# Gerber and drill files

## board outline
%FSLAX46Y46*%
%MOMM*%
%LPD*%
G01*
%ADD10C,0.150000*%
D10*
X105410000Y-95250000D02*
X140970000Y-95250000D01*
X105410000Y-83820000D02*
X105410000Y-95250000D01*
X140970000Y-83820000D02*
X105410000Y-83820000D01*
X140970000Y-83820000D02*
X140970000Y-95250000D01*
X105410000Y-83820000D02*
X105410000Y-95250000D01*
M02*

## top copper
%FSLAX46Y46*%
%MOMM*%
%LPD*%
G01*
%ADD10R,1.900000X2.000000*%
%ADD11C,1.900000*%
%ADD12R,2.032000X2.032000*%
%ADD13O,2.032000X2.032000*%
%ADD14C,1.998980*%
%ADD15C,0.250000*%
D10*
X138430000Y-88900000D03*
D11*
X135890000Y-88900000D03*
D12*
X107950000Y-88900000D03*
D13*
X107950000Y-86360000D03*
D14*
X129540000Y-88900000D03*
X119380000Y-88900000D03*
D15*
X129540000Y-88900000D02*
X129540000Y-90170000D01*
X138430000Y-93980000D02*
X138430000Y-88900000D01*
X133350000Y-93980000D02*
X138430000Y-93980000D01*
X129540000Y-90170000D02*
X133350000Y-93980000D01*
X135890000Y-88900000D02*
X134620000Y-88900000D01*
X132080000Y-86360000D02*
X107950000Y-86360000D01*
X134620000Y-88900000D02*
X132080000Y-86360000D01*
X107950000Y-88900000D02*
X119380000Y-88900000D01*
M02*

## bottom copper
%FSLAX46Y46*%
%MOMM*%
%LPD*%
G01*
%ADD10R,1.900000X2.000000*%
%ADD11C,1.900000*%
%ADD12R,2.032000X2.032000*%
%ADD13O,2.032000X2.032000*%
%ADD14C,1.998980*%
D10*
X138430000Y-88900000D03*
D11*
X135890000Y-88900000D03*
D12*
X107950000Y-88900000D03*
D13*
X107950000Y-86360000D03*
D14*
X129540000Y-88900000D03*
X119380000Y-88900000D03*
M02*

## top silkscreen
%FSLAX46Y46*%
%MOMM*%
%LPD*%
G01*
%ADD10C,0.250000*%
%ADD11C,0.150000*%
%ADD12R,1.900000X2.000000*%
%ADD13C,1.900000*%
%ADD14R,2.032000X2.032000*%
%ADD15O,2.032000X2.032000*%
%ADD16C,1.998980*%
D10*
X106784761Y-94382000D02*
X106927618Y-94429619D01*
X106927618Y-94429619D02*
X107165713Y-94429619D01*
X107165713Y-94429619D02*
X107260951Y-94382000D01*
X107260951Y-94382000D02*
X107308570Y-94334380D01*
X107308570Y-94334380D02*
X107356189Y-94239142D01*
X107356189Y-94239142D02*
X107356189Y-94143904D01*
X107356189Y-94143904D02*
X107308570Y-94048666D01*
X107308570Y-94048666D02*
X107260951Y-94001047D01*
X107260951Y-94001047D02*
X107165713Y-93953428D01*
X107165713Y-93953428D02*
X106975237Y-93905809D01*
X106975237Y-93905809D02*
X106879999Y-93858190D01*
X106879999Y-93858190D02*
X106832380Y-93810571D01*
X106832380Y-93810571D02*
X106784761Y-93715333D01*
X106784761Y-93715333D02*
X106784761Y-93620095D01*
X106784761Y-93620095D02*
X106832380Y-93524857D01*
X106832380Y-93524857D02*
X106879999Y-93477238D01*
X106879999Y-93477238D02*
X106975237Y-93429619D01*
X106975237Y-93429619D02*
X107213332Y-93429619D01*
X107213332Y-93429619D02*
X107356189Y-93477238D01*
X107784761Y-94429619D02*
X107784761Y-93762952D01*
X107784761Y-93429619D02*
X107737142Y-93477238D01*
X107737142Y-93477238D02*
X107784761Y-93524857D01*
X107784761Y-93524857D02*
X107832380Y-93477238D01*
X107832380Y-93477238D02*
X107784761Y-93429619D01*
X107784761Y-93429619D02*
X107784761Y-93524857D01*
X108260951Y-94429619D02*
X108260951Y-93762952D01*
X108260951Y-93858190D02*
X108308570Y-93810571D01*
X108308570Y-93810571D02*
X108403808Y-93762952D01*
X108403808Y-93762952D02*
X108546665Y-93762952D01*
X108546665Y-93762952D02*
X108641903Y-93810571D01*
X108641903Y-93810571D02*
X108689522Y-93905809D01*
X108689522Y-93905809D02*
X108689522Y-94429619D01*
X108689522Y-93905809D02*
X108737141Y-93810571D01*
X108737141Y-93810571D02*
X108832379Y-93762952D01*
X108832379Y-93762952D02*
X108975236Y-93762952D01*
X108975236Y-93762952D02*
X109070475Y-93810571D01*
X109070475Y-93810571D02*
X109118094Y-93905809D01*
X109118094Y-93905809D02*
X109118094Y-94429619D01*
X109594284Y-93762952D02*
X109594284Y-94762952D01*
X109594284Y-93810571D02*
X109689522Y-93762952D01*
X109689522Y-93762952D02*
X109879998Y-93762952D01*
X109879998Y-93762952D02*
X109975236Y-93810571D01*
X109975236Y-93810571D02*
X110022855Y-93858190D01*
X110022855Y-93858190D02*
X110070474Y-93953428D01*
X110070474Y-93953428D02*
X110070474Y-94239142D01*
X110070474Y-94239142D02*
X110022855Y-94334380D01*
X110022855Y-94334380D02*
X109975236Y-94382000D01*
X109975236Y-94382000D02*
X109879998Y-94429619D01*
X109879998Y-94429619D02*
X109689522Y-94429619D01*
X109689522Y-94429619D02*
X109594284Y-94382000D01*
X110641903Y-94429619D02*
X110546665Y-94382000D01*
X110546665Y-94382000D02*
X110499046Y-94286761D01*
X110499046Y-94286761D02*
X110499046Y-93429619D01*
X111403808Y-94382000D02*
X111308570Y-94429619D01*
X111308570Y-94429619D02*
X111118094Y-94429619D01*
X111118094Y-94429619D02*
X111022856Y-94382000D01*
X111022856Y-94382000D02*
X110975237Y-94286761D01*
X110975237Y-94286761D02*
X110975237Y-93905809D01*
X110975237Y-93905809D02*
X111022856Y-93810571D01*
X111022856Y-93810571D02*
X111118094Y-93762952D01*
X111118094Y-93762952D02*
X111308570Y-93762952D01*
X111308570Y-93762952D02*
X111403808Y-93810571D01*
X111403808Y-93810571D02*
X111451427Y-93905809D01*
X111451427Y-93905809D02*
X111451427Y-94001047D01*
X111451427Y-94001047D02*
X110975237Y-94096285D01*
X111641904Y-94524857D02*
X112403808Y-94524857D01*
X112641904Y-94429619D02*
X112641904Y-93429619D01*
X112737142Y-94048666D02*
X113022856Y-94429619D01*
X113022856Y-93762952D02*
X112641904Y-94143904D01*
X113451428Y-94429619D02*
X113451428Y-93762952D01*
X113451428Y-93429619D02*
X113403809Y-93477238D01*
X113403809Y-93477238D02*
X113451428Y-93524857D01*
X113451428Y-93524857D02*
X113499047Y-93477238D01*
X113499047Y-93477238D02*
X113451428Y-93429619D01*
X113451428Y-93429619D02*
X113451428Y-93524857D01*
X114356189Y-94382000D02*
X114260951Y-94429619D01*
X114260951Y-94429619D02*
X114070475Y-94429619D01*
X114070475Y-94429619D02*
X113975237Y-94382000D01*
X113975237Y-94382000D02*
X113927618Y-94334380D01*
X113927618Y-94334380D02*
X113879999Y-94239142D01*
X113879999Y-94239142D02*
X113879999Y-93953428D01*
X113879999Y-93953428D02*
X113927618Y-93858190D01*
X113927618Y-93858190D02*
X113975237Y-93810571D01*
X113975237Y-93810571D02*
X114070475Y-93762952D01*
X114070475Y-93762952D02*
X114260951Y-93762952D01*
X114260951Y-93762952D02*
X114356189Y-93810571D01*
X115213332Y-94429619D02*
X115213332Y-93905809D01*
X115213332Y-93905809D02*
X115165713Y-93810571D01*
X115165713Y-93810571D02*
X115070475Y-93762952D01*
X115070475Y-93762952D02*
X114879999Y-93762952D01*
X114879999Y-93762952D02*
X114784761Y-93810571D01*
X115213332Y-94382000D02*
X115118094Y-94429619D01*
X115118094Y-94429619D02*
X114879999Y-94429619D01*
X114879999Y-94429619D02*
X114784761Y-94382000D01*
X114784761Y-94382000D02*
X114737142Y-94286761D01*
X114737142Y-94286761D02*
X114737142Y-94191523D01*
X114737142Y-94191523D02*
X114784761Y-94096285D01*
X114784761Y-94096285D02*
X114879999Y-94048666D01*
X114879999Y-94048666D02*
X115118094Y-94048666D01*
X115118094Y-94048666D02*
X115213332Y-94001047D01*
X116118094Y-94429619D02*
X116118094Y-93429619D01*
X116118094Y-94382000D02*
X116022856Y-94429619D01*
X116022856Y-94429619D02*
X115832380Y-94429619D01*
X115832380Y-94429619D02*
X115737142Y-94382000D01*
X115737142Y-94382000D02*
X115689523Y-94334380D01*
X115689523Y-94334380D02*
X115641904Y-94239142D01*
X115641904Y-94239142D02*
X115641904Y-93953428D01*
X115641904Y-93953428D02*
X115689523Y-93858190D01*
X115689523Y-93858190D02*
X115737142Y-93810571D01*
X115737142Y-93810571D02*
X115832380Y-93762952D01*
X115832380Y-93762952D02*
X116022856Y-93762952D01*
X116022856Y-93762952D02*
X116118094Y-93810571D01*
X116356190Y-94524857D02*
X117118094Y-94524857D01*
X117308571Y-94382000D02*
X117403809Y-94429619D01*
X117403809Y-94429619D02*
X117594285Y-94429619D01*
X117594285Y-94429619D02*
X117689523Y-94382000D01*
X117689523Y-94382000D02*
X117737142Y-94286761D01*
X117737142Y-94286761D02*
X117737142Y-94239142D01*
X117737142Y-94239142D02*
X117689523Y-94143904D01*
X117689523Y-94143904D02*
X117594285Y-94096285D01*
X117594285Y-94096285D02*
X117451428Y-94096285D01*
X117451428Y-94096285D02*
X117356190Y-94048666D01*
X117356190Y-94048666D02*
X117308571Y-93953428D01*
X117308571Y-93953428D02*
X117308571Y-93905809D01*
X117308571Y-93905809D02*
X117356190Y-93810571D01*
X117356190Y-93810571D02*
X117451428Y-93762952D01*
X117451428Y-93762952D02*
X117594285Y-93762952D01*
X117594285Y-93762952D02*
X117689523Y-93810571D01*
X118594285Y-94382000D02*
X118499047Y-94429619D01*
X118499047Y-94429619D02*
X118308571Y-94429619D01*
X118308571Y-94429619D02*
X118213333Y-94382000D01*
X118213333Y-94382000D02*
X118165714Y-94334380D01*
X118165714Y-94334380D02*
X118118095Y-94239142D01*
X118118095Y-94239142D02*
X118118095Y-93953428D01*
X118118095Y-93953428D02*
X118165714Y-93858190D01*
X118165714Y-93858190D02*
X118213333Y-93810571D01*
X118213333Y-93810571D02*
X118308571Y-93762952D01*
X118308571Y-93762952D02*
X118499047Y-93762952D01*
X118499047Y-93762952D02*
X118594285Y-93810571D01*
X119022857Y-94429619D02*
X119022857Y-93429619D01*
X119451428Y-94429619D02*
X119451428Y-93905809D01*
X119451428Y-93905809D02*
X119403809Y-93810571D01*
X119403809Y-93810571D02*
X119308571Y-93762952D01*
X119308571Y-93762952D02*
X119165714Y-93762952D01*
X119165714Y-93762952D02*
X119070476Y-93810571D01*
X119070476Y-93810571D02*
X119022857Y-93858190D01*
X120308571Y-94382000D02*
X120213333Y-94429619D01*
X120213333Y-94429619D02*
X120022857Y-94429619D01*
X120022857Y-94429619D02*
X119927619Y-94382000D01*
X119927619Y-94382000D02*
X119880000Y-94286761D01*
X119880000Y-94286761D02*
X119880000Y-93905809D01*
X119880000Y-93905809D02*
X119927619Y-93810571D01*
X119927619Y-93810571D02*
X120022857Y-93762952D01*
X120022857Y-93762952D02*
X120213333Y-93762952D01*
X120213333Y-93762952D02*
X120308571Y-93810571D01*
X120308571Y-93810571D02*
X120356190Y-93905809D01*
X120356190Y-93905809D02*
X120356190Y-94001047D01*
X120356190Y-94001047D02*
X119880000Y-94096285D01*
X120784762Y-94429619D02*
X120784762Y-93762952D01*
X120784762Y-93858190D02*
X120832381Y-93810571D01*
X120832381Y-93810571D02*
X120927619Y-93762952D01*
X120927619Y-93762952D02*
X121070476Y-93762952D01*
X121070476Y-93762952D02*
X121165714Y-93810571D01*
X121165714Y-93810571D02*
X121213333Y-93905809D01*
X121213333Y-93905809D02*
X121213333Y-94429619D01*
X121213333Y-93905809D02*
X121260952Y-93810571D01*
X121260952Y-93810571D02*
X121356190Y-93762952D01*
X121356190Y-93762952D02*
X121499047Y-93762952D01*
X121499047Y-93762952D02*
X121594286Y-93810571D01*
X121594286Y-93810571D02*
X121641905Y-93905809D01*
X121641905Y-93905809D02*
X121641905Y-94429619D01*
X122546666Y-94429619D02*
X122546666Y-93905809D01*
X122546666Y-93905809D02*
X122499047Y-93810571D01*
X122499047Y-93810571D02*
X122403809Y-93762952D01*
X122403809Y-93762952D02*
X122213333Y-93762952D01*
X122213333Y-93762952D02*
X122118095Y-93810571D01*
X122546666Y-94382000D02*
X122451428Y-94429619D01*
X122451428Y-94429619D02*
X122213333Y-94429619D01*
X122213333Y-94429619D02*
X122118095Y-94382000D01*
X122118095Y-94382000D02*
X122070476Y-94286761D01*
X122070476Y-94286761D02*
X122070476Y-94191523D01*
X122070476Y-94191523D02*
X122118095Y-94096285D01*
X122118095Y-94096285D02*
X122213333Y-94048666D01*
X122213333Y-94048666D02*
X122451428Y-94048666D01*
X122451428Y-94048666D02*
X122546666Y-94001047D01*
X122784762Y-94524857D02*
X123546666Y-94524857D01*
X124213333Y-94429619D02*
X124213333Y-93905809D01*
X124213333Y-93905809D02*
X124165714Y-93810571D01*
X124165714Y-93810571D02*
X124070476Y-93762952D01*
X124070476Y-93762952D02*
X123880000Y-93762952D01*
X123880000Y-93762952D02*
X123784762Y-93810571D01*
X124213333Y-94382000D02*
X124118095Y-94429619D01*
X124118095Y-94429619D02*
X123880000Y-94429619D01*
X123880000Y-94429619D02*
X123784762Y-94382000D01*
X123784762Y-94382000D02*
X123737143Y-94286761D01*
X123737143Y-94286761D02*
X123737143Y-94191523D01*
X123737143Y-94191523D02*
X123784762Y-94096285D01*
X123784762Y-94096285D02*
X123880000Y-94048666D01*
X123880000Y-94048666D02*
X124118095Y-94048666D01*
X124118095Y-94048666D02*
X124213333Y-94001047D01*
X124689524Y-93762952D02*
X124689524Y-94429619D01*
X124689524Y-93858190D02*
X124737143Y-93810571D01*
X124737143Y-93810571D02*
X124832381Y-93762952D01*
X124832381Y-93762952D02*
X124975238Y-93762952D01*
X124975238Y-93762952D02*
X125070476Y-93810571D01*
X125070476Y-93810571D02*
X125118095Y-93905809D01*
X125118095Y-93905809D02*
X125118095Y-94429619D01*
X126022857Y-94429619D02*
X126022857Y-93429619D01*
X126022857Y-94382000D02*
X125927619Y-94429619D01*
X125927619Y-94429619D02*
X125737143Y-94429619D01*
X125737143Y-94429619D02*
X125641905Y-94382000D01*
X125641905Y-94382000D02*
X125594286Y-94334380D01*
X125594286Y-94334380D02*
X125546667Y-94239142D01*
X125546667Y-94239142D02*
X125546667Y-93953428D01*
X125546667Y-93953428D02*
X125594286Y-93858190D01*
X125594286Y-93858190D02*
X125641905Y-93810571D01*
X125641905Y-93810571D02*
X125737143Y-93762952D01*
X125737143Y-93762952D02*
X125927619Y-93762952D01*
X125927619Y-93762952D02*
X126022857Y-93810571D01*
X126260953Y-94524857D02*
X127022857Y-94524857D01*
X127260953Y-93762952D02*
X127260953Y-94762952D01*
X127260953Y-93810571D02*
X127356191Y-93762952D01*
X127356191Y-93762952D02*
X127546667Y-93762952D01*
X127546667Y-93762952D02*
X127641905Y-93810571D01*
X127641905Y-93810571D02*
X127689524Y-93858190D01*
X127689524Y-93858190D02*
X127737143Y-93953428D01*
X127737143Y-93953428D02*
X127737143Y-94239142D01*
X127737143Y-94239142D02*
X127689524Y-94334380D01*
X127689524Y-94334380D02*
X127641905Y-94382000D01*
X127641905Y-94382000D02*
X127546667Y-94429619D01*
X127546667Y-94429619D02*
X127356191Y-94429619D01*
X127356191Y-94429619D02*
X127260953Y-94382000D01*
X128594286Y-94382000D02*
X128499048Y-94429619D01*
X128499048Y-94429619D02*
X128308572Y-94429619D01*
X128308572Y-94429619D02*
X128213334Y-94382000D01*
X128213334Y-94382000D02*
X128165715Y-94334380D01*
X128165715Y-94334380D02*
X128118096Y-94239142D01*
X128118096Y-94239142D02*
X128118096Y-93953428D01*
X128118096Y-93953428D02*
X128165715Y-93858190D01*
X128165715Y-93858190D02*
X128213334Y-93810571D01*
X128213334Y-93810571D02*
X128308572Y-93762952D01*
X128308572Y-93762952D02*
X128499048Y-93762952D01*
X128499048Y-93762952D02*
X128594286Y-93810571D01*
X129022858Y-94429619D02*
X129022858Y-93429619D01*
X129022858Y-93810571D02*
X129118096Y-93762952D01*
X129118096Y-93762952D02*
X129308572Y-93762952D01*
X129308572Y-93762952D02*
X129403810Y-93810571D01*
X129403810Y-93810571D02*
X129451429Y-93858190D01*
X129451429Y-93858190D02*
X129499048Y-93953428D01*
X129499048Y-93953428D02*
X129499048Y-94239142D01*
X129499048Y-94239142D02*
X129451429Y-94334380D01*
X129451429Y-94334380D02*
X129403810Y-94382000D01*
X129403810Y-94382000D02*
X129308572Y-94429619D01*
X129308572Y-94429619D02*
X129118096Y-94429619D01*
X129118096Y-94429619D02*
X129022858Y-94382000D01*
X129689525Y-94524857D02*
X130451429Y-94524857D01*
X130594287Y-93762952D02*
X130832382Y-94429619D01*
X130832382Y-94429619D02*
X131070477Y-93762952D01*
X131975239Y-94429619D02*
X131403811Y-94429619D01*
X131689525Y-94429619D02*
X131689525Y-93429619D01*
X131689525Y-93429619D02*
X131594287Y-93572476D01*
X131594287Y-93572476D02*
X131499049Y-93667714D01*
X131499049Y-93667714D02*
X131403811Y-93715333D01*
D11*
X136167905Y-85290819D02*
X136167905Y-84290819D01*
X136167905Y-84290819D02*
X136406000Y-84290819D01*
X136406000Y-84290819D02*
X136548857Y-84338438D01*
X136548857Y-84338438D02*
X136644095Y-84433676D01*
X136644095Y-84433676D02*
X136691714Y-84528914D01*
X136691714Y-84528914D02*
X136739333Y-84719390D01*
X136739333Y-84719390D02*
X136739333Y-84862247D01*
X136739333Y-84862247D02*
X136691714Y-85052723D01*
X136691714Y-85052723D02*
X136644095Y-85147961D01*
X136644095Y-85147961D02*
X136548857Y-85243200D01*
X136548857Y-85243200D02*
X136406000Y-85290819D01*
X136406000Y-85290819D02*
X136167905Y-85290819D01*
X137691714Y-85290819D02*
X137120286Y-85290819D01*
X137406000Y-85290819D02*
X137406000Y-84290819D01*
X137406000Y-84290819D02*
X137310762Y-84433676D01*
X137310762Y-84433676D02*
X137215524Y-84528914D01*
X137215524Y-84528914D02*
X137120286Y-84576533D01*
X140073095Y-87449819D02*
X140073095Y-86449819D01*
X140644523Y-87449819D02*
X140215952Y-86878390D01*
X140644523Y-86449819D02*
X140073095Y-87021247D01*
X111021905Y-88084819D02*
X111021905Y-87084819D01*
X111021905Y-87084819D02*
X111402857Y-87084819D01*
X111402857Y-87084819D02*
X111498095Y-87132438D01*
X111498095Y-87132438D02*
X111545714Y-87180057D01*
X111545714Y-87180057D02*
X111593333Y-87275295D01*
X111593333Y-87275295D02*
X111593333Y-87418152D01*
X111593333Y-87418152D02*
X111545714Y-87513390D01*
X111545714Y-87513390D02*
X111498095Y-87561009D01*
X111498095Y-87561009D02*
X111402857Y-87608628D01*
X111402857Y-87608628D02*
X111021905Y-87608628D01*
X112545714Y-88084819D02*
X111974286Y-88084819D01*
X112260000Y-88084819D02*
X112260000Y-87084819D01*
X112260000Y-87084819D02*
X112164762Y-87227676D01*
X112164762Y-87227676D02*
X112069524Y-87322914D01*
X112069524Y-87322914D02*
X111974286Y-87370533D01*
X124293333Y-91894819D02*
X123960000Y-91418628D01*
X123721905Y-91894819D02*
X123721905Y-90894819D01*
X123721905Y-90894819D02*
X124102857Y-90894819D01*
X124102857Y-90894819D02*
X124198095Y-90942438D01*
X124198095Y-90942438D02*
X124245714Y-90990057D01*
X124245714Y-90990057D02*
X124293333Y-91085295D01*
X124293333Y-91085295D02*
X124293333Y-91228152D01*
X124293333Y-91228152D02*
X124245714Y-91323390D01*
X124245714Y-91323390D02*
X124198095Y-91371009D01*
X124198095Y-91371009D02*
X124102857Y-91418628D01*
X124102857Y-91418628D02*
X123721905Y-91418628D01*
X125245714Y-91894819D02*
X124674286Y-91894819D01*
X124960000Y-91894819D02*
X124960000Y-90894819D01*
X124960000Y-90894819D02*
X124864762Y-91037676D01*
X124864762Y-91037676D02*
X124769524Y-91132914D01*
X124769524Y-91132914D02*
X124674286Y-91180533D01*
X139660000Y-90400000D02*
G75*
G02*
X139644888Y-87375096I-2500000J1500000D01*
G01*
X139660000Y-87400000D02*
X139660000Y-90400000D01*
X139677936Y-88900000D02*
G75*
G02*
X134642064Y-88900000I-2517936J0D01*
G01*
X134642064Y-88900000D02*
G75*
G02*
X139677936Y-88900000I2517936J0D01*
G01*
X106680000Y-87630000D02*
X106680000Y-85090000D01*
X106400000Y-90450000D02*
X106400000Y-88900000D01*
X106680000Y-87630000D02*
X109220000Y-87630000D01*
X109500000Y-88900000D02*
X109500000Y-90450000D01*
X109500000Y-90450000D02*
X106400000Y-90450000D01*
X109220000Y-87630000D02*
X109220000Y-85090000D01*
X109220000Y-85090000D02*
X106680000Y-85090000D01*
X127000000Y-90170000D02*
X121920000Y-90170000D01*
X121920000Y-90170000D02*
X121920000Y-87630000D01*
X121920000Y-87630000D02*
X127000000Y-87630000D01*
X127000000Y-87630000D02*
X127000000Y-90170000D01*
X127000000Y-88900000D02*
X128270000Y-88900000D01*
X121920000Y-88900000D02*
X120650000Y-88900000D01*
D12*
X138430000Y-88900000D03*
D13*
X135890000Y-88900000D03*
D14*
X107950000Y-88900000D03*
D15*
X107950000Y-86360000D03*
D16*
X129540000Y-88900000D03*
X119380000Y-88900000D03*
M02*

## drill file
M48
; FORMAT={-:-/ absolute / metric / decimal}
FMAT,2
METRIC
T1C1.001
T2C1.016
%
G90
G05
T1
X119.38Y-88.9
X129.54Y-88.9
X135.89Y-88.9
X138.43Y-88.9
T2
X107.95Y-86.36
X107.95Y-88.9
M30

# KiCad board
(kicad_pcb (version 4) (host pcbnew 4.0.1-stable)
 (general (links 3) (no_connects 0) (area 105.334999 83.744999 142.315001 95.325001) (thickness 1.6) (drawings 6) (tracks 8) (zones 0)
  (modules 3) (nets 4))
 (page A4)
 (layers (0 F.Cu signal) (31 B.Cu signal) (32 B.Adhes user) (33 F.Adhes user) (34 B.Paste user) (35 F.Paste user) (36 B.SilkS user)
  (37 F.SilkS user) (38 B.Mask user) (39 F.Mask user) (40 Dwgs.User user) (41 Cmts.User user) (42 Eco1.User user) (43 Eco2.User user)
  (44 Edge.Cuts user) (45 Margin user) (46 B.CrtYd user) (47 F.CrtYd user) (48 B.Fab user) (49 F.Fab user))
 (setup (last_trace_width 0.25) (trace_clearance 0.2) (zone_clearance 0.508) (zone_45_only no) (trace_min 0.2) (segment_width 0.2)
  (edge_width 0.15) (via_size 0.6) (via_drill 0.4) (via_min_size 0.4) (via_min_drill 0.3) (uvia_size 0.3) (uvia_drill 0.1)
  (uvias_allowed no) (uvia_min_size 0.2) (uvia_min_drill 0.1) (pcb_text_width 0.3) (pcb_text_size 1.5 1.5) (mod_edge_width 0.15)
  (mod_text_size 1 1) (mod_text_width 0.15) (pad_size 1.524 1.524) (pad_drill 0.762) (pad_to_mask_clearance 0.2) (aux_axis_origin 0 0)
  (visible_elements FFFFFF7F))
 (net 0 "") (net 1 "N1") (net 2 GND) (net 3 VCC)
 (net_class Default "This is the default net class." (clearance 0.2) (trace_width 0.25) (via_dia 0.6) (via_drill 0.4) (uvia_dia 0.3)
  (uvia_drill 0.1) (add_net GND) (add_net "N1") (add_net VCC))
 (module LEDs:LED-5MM (layer F.Cu) (at 138.43 88.9 180)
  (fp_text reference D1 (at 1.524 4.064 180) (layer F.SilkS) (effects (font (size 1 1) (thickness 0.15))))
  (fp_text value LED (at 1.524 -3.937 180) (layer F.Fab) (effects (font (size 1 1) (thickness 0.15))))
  (fp_arc (start 1.27 0) (end -1.23 -1.5) (angle 297.5) (layer F.SilkS) (width 0.15))
  (fp_line (start -1.23 1.5) (end -1.23 -1.5) (layer F.SilkS) (width 0.15))
  (fp_circle (center 1.27 0) (end 0.97 -2.5) (layer F.SilkS) (width 0.15))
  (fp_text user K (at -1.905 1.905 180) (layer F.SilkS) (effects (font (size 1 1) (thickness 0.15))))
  (pad 1 thru_hole rect (at 0 0 270) (size 2 1.9) (drill 1.00076) (layers *.Cu *.Mask F.SilkS) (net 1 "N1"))
  (pad 2 thru_hole circle (at 2.54 0 180) (size 1.9 1.9) (drill 1.00076) (layers *.Cu *.Mask F.SilkS) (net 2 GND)))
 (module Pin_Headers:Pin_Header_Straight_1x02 (layer F.Cu) (at 107.95 88.9 180)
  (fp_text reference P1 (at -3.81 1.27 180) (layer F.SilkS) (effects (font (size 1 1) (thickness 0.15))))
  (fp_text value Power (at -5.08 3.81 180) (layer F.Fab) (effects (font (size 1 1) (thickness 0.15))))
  (fp_line (start 1.27 1.27) (end 1.27 3.81) (layer F.SilkS) (width 0.15))
  (fp_line (start 1.55 -1.55) (end 1.55 0) (layer F.SilkS) (width 0.15))
  (fp_line (start 1.27 1.27) (end -1.27 1.27) (layer F.SilkS) (width 0.15))
  (fp_line (start -1.55 0) (end -1.55 -1.55) (layer F.SilkS) (width 0.15))
  (fp_line (start -1.55 -1.55) (end 1.55 -1.55) (layer F.SilkS) (width 0.15))
  (fp_line (start -1.27 1.27) (end -1.27 3.81) (layer F.SilkS) (width 0.15))
  (fp_line (start -1.27 3.81) (end 1.27 3.81) (layer F.SilkS) (width 0.15))
  (pad 1 thru_hole rect (at 0 0 180) (size 2.032 2.032) (drill 1.016) (layers *.Cu *.Mask F.SilkS) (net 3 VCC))
  (pad 2 thru_hole oval (at 0 2.54 180) (size 2.032 2.032) (drill 1.016) (layers *.Cu *.Mask F.SilkS) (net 2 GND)))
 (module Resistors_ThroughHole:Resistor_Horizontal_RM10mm (layer F.Cu) (at 124.46 88.9 180)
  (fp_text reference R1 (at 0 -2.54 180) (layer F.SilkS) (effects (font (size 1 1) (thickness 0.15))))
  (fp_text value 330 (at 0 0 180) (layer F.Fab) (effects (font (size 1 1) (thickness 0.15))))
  (fp_line (start -2.54 -1.27) (end 2.54 -1.27) (layer F.SilkS) (width 0.15))
  (fp_line (start 2.54 -1.27) (end 2.54 1.27) (layer F.SilkS) (width 0.15))
  (fp_line (start 2.54 1.27) (end -2.54 1.27) (layer F.SilkS) (width 0.15))
  (fp_line (start -2.54 1.27) (end -2.54 -1.27) (layer F.SilkS) (width 0.15))
  (fp_line (start -2.54 0) (end -3.81 0) (layer F.SilkS) (width 0.15))
  (fp_line (start 2.54 0) (end 3.81 0) (layer F.SilkS) (width 0.15))
  (pad 1 thru_hole circle (at -5.08 0 180) (size 1.99898 1.99898) (drill 1.00076) (layers *.Cu *.SilkS *.Mask) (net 1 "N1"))
  (pad 2 thru_hole circle (at 5.08 0 180) (size 1.99898 1.99898) (drill 1.00076) (layers *.Cu *.SilkS *.Mask) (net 3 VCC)))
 (gr_line (start 105.41 95.25) (end 140.97 95.25) (angle 90) (layer Edge.Cuts) (width 0.15))
 (gr_line (start 105.41 83.82) (end 105.41 95.25) (angle 90) (layer Edge.Cuts) (width 0.15))
 (gr_line (start 140.97 83.82) (end 105.41 83.82) (angle 90) (layer Edge.Cuts) (width 0.15))
 (gr_line (start 140.97 83.82) (end 140.97 95.25) (angle 90) (layer Edge.Cuts) (width 0.15))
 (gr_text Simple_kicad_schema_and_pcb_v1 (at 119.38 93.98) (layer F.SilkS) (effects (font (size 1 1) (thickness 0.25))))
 (gr_line (start 105.41 83.82) (end 105.41 95.25) (angle 90) (layer Edge.Cuts) (width 0.15))
 (segment (start 129.54 88.9) (end 129.54 90.17) (width 0.25) (layer F.Cu) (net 1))
 (segment (start 138.43 93.98) (end 138.43 88.9) (width 0.25) (layer F.Cu) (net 1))
 (segment (start 133.35 93.98) (end 138.43 93.98) (width 0.25) (layer F.Cu) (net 1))
 (segment (start 129.54 90.17) (end 133.35 93.98) (width 0.25) (layer F.Cu) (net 1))
 (segment (start 135.89 88.9) (end 134.62 88.9) (width 0.25) (layer F.Cu) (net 2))
 (segment (start 132.08 86.36) (end 107.95 86.36) (width 0.25) (layer F.Cu) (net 2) (status 20))
 (segment (start 134.62 88.9) (end 132.08 86.36) (width 0.25) (layer F.Cu) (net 2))
 (segment (start 107.95 88.9) (end 119.38 88.9) (width 0.25) (layer F.Cu) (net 3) (status 10)))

